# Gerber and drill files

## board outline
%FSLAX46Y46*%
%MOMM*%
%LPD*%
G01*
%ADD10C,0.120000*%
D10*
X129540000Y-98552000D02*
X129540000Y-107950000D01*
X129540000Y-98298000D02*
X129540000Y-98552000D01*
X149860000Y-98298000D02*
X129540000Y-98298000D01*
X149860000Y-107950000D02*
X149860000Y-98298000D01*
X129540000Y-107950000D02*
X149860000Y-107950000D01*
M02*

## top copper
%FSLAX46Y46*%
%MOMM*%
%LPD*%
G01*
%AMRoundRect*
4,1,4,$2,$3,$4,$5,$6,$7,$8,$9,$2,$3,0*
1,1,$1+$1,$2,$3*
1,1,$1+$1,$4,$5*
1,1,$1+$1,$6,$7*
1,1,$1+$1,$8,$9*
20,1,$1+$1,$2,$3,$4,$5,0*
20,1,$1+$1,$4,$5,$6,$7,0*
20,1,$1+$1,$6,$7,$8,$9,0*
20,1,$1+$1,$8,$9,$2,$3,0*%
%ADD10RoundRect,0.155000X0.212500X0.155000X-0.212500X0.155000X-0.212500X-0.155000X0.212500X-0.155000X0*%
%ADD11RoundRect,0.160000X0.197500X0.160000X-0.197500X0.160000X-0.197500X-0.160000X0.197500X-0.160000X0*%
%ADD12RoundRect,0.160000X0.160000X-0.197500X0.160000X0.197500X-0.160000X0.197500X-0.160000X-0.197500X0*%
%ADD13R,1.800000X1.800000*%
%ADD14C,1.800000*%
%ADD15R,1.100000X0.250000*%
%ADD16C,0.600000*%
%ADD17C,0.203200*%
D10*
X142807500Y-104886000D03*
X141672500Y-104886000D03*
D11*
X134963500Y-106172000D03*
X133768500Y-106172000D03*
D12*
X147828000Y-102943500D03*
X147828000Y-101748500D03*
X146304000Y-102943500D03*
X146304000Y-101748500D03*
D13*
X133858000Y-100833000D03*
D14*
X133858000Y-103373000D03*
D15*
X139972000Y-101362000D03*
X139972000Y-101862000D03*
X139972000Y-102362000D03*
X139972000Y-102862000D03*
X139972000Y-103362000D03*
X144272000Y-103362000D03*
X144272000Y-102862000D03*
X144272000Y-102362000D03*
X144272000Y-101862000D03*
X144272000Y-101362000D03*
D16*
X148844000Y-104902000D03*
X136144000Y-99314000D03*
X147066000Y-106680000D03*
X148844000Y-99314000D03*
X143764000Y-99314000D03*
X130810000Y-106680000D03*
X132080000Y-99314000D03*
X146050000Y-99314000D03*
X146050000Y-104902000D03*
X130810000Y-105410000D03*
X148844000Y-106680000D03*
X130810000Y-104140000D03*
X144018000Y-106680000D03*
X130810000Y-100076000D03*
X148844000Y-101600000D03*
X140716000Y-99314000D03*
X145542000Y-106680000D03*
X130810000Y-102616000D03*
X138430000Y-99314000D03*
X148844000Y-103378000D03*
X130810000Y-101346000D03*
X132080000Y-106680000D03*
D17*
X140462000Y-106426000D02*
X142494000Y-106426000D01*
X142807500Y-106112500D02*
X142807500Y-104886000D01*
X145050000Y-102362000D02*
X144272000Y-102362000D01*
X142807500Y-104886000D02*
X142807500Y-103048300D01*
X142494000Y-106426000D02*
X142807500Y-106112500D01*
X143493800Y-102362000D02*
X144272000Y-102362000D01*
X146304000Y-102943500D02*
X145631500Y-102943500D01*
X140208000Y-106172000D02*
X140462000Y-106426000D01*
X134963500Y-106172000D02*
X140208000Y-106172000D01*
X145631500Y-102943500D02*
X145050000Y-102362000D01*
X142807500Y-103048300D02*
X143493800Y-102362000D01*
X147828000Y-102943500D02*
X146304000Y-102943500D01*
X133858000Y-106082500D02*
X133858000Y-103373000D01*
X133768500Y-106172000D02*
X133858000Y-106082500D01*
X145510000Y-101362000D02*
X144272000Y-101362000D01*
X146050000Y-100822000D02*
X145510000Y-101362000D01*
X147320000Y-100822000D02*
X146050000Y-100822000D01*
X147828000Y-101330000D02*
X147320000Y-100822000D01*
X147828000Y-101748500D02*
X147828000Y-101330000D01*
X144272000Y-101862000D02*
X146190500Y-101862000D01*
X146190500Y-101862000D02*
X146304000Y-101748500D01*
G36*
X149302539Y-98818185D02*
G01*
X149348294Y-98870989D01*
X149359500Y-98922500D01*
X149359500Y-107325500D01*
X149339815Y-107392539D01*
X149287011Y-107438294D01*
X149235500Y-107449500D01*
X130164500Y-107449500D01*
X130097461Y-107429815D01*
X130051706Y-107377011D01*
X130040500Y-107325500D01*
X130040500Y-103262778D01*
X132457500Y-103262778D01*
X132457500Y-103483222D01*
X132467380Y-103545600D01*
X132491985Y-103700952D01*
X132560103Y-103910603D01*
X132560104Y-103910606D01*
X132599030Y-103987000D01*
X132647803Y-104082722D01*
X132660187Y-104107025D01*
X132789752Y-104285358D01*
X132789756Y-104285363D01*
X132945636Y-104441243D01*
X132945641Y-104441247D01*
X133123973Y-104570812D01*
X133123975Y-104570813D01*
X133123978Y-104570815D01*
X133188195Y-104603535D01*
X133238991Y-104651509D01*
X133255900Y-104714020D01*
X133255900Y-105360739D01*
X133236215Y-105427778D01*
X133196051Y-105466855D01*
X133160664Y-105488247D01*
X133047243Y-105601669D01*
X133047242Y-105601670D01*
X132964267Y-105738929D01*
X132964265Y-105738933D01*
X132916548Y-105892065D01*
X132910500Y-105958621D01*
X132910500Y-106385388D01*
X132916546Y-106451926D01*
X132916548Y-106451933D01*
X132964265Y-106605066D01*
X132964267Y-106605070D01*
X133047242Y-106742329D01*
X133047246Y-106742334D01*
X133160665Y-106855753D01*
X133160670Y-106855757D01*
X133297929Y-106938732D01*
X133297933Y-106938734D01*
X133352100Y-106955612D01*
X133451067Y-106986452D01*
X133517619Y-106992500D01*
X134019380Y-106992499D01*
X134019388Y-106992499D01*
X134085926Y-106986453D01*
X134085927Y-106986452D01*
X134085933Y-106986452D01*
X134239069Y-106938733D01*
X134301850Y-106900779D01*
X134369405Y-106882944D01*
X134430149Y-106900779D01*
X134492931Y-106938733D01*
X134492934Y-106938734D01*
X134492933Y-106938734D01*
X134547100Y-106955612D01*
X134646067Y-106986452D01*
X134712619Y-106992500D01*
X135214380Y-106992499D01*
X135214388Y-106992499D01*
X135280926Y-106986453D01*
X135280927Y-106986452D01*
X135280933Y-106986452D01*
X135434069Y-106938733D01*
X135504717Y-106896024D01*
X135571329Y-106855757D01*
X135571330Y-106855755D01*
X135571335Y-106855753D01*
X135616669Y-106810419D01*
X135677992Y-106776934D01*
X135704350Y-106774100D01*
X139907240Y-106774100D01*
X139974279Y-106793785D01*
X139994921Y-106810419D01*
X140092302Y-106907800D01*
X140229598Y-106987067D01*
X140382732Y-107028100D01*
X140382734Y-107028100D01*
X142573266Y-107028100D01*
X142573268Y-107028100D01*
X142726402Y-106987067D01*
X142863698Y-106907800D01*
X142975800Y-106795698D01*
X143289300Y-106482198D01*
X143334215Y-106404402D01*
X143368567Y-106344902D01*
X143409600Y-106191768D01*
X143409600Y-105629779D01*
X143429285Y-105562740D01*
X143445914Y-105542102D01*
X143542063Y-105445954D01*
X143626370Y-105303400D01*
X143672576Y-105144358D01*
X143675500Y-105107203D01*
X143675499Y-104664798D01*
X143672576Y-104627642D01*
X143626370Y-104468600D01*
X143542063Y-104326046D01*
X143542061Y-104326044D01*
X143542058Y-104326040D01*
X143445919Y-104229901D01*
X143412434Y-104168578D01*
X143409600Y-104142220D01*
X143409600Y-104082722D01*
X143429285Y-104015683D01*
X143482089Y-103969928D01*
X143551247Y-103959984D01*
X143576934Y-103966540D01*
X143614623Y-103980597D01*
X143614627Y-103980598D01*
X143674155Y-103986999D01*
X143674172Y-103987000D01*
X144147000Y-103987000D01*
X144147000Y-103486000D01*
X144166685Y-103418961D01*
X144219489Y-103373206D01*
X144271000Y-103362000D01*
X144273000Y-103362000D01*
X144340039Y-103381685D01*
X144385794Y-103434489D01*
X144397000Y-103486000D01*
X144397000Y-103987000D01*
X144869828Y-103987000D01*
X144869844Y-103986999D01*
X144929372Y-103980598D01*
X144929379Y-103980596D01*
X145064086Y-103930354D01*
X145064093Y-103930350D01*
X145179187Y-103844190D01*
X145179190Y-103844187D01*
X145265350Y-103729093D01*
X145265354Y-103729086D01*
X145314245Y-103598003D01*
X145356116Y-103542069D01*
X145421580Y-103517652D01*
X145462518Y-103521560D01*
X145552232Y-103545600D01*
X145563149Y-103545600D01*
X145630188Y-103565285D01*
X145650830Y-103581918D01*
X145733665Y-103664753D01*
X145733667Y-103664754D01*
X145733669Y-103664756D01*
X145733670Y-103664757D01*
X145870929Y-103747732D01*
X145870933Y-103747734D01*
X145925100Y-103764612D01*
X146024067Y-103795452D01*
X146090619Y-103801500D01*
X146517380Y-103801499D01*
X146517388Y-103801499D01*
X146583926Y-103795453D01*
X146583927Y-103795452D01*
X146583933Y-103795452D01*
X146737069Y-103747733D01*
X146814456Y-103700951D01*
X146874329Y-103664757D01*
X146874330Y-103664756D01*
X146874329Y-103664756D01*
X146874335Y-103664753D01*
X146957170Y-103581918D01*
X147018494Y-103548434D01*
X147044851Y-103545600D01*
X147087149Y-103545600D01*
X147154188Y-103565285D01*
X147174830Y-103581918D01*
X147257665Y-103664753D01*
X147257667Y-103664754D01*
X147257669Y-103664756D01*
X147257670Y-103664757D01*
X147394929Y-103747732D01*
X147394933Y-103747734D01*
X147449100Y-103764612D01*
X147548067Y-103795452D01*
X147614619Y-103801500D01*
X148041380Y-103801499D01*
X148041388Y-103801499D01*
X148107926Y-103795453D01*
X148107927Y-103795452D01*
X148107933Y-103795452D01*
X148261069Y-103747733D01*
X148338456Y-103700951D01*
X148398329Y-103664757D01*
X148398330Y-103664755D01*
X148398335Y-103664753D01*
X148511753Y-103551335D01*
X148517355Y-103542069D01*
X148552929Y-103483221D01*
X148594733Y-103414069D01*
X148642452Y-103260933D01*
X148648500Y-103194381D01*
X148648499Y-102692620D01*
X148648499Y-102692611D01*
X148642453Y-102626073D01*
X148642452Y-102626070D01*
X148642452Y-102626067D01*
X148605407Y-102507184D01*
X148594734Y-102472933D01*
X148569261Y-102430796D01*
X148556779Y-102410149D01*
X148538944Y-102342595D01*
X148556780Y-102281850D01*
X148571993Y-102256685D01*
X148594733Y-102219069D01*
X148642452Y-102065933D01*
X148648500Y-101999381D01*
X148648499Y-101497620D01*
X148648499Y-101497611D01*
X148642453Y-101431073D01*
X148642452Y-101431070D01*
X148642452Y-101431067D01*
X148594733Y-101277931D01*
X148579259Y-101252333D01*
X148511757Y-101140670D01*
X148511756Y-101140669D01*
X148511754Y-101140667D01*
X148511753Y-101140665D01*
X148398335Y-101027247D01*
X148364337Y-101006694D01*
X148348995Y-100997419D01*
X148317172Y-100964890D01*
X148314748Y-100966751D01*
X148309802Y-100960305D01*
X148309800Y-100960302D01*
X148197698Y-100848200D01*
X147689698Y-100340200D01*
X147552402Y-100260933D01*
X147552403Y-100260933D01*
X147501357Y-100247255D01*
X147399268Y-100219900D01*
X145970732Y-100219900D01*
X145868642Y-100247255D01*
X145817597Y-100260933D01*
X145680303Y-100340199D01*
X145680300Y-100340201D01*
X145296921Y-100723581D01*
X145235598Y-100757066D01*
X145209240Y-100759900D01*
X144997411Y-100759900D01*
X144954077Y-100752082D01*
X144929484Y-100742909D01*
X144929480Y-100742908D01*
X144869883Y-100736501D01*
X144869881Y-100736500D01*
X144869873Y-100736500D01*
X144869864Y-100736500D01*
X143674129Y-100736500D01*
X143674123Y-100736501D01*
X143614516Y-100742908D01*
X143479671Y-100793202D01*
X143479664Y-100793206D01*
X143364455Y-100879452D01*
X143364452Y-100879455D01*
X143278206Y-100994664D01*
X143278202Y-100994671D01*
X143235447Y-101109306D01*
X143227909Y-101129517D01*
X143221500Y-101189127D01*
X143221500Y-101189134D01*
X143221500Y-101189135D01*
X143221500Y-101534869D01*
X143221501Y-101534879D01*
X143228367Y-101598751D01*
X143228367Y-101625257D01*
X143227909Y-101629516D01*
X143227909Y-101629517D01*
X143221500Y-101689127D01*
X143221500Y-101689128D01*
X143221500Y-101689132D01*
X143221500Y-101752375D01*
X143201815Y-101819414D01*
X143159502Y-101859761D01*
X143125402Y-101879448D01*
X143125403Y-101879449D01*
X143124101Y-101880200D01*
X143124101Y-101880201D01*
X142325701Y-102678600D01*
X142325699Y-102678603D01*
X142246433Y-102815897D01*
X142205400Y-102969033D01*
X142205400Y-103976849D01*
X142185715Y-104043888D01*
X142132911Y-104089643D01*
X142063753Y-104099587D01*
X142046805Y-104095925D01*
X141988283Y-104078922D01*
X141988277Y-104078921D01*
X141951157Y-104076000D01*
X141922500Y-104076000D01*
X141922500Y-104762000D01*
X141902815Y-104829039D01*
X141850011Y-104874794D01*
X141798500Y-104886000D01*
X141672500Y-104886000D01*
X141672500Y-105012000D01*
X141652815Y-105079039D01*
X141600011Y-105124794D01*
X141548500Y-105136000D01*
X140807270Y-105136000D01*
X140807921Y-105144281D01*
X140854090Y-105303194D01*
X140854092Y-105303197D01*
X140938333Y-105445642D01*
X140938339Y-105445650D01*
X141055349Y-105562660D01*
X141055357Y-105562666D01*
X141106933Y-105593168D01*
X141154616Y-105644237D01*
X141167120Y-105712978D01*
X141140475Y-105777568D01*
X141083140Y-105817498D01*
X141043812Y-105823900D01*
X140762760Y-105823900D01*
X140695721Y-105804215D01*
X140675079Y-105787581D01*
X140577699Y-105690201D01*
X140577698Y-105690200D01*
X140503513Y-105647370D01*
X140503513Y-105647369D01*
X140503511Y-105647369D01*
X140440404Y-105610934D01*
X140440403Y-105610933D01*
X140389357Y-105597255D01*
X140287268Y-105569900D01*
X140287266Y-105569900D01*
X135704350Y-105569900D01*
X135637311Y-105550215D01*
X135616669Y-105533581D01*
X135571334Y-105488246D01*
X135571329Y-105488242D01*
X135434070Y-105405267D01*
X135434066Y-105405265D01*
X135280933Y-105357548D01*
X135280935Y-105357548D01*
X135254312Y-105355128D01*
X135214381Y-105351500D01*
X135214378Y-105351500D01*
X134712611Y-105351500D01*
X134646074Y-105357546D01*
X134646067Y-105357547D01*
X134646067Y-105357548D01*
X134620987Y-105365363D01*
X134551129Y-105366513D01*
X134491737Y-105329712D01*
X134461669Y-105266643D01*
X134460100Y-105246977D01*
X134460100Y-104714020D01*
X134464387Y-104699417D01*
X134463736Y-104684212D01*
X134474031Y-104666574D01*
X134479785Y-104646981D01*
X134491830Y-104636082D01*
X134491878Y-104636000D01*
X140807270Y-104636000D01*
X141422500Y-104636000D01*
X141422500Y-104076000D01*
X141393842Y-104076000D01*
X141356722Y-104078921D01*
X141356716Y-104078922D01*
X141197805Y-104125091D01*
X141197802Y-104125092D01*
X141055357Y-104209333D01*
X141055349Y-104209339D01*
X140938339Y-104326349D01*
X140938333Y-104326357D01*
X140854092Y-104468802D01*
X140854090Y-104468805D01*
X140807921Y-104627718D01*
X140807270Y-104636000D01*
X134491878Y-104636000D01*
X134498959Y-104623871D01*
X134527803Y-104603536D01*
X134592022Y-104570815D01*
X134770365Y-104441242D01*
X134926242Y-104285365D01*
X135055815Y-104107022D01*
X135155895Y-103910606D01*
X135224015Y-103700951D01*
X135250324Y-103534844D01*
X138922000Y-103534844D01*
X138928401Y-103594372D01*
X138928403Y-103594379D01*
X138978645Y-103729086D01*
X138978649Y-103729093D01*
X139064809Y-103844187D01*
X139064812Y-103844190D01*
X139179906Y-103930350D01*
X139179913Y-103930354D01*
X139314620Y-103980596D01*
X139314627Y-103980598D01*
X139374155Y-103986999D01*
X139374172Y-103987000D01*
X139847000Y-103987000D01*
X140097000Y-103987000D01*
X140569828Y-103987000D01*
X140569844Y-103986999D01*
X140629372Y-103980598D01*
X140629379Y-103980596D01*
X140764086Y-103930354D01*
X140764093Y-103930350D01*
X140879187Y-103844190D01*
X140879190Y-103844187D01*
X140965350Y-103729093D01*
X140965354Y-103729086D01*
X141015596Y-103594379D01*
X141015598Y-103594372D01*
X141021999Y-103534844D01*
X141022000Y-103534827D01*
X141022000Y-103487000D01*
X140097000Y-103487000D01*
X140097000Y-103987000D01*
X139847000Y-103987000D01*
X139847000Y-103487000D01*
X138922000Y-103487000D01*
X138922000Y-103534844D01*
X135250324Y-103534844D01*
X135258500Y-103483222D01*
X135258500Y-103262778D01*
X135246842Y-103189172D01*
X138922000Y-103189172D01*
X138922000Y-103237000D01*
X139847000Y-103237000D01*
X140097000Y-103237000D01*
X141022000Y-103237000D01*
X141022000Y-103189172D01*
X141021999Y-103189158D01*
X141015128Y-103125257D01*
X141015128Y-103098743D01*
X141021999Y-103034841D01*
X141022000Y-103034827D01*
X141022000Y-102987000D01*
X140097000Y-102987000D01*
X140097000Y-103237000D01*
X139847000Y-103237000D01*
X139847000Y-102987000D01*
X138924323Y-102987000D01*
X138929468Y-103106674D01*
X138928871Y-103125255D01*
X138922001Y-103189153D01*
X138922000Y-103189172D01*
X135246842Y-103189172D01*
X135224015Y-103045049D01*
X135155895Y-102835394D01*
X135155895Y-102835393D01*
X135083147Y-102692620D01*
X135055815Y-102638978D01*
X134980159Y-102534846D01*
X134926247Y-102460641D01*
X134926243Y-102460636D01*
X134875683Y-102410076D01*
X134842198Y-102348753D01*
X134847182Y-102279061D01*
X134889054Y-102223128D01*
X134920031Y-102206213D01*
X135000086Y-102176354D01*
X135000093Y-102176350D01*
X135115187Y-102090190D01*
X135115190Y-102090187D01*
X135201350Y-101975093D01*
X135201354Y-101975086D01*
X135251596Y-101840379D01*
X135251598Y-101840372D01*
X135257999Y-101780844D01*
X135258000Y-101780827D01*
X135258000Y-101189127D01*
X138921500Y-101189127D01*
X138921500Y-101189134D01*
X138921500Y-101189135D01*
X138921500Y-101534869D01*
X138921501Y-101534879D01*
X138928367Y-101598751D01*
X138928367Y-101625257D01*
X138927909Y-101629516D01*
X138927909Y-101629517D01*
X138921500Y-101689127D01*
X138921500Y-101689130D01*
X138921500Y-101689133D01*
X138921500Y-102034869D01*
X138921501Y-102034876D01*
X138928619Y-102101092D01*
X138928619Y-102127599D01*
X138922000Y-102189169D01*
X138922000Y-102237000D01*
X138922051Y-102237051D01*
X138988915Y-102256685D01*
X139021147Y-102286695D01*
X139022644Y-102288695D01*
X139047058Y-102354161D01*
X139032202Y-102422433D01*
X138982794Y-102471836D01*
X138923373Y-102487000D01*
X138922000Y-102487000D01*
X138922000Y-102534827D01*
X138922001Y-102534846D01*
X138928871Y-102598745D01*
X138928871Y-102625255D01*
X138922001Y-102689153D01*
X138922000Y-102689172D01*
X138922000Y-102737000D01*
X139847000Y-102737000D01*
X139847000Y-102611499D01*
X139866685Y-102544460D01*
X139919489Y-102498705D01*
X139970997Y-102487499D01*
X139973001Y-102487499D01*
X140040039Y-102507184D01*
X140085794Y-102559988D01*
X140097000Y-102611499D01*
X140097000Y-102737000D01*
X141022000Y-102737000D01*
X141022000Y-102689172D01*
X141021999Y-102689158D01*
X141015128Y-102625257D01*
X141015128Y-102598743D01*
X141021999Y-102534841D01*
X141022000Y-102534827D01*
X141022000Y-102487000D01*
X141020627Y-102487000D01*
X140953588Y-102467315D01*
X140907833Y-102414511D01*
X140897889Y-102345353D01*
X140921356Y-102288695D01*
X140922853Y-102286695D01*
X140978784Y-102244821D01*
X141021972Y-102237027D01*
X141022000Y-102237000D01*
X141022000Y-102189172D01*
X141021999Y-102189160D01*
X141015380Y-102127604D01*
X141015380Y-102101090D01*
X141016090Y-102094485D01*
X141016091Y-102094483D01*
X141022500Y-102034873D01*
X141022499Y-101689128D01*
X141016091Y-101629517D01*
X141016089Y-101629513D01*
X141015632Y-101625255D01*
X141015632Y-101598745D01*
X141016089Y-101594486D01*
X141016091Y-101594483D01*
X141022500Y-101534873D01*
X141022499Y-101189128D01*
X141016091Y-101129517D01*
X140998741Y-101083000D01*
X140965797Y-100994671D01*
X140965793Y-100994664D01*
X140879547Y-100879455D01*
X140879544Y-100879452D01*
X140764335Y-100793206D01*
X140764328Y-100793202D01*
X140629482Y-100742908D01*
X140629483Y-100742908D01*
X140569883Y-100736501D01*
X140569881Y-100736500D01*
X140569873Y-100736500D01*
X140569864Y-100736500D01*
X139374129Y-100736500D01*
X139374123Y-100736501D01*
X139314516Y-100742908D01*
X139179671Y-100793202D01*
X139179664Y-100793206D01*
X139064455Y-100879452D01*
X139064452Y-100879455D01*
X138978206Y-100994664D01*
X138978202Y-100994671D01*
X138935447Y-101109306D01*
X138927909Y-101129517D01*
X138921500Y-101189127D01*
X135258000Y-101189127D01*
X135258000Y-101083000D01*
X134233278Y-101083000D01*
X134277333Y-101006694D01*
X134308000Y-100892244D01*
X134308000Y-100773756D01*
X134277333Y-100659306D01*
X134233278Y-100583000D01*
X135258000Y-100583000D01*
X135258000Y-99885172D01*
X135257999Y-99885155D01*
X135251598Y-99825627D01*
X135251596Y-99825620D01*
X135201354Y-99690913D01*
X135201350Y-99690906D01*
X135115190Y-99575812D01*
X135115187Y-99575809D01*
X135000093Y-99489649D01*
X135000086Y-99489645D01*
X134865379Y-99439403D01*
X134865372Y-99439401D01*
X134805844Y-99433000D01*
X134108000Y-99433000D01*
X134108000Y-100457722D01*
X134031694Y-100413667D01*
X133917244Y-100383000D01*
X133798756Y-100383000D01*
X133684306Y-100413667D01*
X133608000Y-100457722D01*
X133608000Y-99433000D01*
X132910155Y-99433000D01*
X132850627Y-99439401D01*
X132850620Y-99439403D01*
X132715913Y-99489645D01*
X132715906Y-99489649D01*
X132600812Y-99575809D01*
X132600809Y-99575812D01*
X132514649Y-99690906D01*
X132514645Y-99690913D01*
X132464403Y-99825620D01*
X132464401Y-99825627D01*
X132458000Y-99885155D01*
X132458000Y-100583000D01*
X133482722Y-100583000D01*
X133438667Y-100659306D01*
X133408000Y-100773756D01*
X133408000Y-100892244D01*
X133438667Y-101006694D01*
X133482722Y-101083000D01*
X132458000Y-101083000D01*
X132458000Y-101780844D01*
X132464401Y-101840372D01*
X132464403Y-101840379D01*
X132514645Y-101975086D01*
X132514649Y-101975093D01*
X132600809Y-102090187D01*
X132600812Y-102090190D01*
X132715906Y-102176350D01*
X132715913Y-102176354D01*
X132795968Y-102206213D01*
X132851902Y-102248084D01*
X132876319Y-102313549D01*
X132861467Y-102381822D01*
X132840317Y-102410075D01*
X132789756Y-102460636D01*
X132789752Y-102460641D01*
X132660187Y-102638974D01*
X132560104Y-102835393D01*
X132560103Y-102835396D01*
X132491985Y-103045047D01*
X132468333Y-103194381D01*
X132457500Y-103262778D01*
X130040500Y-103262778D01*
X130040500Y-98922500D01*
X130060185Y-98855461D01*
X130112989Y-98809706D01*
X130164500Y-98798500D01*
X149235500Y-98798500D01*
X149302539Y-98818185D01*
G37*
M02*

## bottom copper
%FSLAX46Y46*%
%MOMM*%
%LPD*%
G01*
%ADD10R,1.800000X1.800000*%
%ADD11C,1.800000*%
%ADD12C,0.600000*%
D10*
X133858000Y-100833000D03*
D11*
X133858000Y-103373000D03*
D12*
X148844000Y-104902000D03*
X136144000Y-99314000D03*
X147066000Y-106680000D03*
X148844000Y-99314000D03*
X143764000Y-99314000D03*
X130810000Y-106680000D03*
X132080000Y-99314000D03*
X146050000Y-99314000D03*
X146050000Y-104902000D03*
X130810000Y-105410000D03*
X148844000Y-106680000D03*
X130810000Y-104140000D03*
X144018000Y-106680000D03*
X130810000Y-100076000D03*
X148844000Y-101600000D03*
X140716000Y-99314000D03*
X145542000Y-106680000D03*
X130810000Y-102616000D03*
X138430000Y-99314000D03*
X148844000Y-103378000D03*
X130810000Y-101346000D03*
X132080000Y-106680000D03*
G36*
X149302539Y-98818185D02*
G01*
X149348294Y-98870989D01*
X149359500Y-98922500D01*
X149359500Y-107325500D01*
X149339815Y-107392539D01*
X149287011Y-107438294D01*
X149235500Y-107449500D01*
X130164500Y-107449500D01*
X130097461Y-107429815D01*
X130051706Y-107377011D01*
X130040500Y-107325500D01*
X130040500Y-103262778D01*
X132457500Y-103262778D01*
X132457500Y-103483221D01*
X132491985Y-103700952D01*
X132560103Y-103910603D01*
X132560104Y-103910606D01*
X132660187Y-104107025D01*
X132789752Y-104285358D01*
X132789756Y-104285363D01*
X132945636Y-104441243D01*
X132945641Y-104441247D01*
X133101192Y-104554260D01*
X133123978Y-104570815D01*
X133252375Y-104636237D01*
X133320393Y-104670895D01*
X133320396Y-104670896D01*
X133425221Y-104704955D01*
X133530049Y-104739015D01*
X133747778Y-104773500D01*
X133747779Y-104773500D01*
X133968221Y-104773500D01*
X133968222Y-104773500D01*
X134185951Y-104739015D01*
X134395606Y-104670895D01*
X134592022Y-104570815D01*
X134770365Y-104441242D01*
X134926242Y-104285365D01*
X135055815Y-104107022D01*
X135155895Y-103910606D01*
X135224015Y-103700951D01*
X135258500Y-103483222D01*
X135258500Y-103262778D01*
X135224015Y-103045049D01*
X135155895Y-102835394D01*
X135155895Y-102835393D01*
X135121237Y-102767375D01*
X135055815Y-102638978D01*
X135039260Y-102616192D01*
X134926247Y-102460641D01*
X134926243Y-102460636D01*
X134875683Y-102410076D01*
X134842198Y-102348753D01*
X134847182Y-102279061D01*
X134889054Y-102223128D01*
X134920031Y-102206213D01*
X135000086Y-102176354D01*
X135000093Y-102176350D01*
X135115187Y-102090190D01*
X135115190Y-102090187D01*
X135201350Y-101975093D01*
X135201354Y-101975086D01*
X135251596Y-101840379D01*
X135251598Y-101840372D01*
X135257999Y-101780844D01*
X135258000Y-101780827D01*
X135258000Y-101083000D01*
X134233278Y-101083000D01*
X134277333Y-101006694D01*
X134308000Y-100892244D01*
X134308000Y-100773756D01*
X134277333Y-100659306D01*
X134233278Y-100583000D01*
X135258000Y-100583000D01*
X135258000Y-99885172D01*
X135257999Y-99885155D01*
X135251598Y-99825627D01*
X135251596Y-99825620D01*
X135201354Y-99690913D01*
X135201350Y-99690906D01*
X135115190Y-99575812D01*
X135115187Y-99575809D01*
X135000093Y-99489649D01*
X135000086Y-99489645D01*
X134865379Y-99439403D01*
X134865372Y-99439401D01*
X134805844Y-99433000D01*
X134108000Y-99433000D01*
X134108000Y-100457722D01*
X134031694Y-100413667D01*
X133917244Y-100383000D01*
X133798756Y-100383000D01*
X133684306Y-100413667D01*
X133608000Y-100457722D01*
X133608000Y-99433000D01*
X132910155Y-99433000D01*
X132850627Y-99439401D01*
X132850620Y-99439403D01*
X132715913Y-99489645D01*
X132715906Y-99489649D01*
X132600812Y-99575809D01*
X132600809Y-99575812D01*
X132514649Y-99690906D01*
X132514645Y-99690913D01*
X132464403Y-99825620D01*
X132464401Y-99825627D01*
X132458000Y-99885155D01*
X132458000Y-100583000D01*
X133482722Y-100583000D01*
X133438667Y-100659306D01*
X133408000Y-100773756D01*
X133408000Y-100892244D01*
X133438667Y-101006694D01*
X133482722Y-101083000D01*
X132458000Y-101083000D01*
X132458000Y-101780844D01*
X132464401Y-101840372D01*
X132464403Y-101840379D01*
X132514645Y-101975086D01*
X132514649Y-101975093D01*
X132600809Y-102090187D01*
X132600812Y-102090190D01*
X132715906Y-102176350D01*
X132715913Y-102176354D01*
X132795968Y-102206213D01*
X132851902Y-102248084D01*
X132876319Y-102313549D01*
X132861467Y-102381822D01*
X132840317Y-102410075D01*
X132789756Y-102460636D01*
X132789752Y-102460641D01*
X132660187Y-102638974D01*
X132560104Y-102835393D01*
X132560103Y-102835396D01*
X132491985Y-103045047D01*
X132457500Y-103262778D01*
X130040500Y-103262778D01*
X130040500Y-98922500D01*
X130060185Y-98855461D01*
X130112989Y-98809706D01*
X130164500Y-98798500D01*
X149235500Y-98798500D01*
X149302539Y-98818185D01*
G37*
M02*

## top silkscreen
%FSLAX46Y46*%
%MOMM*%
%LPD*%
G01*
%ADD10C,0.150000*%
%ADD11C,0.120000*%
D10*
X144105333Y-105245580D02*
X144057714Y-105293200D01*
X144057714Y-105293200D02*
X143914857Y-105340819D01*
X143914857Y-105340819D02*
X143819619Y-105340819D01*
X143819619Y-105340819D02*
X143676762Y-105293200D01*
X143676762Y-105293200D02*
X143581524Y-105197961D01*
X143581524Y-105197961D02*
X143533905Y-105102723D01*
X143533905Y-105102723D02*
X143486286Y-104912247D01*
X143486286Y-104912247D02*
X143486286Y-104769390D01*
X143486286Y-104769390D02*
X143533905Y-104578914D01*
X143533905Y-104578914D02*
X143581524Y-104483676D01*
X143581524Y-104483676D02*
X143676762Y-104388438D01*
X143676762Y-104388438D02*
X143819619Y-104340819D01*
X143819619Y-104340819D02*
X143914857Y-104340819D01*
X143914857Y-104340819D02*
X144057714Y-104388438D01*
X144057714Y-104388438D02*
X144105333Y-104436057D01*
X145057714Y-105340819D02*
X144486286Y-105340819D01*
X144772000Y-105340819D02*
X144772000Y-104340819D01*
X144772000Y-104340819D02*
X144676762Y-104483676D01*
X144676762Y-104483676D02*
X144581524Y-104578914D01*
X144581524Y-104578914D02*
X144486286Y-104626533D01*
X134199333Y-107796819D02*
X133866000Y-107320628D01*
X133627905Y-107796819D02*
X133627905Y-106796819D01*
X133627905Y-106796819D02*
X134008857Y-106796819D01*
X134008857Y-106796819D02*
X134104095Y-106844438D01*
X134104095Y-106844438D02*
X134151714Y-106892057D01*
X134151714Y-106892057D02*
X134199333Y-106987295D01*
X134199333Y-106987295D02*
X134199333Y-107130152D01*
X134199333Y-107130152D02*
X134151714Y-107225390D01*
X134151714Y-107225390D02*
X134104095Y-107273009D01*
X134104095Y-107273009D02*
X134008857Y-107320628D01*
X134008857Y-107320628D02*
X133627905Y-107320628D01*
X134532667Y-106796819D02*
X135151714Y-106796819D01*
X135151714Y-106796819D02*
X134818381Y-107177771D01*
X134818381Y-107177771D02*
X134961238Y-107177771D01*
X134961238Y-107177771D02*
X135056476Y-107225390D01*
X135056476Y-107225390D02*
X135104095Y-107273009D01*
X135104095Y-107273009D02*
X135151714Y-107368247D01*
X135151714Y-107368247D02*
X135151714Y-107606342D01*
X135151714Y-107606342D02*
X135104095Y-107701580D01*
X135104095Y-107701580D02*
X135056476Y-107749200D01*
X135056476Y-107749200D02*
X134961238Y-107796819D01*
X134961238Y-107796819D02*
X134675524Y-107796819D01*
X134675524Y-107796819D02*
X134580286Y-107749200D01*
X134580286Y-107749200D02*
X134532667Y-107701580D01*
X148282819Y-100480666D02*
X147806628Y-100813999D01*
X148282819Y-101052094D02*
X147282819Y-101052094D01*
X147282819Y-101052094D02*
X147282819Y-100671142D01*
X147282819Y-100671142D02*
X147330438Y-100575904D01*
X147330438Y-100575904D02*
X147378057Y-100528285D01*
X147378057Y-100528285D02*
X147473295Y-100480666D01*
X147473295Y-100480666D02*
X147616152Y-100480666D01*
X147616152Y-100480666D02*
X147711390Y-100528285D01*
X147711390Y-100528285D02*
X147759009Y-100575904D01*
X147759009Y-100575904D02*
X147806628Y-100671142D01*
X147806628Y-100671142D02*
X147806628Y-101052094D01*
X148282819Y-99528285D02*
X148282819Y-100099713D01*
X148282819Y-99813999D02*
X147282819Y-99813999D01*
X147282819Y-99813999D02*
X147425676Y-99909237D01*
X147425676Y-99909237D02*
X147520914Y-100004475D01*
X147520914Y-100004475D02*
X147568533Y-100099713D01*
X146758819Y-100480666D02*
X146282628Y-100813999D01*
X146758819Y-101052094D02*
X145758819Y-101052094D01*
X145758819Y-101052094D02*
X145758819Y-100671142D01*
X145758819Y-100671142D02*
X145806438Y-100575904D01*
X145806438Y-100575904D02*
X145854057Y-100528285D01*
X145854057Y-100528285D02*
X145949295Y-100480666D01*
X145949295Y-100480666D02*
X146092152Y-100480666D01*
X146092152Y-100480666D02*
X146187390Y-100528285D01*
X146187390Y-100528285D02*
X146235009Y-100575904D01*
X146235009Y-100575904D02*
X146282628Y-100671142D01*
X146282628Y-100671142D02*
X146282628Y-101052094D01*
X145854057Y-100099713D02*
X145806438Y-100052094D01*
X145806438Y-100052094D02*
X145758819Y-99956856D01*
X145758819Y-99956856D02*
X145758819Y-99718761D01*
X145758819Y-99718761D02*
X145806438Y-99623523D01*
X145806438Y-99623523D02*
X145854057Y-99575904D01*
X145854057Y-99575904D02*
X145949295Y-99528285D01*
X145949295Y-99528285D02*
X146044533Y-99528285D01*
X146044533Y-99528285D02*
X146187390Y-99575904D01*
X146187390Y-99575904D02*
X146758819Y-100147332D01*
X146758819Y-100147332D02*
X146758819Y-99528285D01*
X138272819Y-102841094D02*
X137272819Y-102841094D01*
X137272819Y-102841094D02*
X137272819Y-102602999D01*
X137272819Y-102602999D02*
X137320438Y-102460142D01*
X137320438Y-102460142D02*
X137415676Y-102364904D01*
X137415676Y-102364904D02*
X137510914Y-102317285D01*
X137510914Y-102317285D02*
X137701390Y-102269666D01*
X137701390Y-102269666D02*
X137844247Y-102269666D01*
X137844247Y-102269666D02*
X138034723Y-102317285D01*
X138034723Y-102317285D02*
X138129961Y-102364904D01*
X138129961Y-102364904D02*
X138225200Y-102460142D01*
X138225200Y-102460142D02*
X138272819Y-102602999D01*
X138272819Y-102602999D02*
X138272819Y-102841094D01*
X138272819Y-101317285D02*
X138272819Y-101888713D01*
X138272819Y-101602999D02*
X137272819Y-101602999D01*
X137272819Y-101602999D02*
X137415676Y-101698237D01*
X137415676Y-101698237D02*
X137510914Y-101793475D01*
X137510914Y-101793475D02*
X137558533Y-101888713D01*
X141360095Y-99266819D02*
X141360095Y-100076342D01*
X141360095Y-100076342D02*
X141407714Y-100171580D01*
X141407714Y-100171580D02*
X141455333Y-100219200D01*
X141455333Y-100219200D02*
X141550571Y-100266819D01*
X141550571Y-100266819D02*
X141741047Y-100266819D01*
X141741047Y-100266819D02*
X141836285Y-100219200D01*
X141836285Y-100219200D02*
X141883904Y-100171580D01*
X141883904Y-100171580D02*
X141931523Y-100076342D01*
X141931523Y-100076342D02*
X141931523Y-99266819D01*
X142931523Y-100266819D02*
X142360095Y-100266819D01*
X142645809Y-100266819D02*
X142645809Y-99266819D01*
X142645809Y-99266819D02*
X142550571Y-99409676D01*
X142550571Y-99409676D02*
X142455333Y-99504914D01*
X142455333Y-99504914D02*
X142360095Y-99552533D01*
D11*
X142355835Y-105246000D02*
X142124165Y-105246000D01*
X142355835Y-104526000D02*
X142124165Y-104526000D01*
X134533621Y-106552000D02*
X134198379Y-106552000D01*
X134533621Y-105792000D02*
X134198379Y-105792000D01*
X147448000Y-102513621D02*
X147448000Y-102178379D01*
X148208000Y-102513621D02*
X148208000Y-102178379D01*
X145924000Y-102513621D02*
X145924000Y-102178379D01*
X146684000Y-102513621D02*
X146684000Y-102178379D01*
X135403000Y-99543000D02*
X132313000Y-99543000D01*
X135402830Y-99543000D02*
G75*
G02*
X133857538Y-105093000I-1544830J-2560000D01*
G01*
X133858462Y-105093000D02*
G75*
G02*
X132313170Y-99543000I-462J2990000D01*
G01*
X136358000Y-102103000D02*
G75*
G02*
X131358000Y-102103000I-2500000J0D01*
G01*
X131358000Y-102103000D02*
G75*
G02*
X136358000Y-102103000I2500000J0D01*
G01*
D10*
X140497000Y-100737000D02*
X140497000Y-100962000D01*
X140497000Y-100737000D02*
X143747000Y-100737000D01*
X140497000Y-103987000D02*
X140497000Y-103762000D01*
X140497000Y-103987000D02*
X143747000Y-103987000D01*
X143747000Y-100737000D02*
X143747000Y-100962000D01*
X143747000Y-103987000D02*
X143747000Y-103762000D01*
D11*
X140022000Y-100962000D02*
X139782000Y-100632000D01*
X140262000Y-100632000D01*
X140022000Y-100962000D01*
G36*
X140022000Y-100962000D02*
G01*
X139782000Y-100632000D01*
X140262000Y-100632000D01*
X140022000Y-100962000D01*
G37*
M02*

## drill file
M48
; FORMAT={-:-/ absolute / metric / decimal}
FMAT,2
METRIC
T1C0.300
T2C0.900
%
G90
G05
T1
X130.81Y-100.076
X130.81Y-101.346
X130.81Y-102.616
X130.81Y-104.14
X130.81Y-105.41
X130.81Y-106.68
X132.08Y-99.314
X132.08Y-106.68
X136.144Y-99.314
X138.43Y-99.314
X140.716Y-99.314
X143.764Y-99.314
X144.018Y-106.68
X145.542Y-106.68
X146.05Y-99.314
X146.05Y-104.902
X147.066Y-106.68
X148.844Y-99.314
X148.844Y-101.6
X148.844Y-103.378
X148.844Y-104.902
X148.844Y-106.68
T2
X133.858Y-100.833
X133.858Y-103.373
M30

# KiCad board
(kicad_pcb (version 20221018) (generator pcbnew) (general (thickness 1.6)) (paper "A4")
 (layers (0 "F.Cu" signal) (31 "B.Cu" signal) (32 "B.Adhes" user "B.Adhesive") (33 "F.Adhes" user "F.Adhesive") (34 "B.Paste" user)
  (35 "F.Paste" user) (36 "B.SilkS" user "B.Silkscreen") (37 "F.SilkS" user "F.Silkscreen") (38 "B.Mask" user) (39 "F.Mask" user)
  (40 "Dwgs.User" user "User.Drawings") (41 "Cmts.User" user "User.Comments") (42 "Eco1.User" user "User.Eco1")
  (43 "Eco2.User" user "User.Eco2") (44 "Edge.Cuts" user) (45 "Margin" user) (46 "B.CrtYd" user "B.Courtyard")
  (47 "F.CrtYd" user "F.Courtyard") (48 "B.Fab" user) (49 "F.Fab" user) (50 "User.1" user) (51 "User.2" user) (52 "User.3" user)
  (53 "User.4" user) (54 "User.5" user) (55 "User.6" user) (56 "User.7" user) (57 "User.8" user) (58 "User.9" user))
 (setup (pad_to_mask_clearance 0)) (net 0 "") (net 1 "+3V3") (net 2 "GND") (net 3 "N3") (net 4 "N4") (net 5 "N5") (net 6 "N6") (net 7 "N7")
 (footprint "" (layer "F.Cu") (at 142.24 104.886 180)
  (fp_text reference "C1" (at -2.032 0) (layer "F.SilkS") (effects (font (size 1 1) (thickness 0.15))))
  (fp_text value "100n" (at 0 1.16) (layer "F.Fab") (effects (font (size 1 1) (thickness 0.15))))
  (fp_line (start -0.115835 -0.36) (end 0.115835 -0.36) (layer "F.SilkS") (stroke (width 0.12) (type solid)))
  (fp_line (start -0.115835 0.36) (end 0.115835 0.36) (layer "F.SilkS") (stroke (width 0.12) (type solid)))
  (pad "1" smd roundrect (at -0.5675 0 180) (size 0.735 0.62) (layers "F.Cu" "F.Paste" "F.Mask") (roundrect_rratio 0.25) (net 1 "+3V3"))
  (pad "2" smd roundrect (at 0.5675 0 180) (size 0.735 0.62) (layers "F.Cu" "F.Paste" "F.Mask") (roundrect_rratio 0.25) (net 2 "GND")))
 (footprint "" (layer "F.Cu") (at 134.366 106.172 180)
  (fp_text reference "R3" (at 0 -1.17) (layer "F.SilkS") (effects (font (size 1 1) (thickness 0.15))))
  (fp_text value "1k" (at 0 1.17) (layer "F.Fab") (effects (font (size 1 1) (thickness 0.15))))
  (fp_line (start -0.167621 -0.38) (end 0.167621 -0.38) (layer "F.SilkS") (stroke (width 0.12) (type solid)))
  (fp_line (start -0.167621 0.38) (end 0.167621 0.38) (layer "F.SilkS") (stroke (width 0.12) (type solid)))
  (pad "1" smd roundrect (at -0.5975 0 180) (size 0.715 0.64) (layers "F.Cu" "F.Paste" "F.Mask") (roundrect_rratio 0.25) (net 1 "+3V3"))
  (pad "2" smd roundrect (at 0.5975 0 180) (size 0.715 0.64) (layers "F.Cu" "F.Paste" "F.Mask") (roundrect_rratio 0.25) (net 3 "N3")))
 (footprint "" (layer "F.Cu") (at 147.828 102.346 90)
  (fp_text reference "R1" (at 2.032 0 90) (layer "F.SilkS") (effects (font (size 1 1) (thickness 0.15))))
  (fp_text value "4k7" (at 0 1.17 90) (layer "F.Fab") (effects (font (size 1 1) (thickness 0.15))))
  (fp_line (start -0.167621 -0.38) (end 0.167621 -0.38) (layer "F.SilkS") (stroke (width 0.12) (type solid)))
  (fp_line (start -0.167621 0.38) (end 0.167621 0.38) (layer "F.SilkS") (stroke (width 0.12) (type solid)))
  (pad "1" smd roundrect (at -0.5975 0 90) (size 0.715 0.64) (layers "F.Cu" "F.Paste" "F.Mask") (roundrect_rratio 0.25) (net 1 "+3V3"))
  (pad "2" smd roundrect (at 0.5975 0 90) (size 0.715 0.64) (layers "F.Cu" "F.Paste" "F.Mask") (roundrect_rratio 0.25) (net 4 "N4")))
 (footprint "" (layer "F.Cu") (at 146.304 102.346 90)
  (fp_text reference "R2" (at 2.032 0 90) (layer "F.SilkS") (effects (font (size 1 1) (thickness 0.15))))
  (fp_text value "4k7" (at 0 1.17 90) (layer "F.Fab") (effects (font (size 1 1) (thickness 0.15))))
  (fp_line (start -0.167621 -0.38) (end 0.167621 -0.38) (layer "F.SilkS") (stroke (width 0.12) (type solid)))
  (fp_line (start -0.167621 0.38) (end 0.167621 0.38) (layer "F.SilkS") (stroke (width 0.12) (type solid)))
  (pad "1" smd roundrect (at -0.5975 0 90) (size 0.715 0.64) (layers "F.Cu" "F.Paste" "F.Mask") (roundrect_rratio 0.25) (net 1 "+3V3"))
  (pad "2" smd roundrect (at 0.5975 0 90) (size 0.715 0.64) (layers "F.Cu" "F.Paste" "F.Mask") (roundrect_rratio 0.25) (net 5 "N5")))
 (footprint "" (layer "F.Cu") (at 133.858 100.833 -90)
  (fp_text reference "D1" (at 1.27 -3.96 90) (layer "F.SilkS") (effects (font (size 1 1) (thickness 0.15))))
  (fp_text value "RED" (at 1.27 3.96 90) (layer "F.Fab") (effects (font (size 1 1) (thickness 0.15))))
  (fp_line (start -1.29 -1.545) (end -1.29 1.545) (layer "F.SilkS") (stroke (width 0.12) (type solid)))
  (fp_arc (start -1.29 -1.54483) (mid 2.072002 -2.880433) (end 4.26 0.000462) (layer "F.SilkS") (stroke (width 0.12) (type solid)))
  (fp_arc (start 4.26 -0.000462) (mid 2.072002 2.880433) (end -1.29 1.54483) (layer "F.SilkS") (stroke (width 0.12) (type solid)))
  (fp_circle (center 1.27 0) (end 3.77 0) (layer "F.SilkS") (stroke (width 0.12) (type solid)) (fill none))
  (pad "1" thru_hole rect (at 0 0 270) (size 1.8 1.8) (drill 0.9) (layers *.Cu *.Mask) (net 2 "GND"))
  (pad "2" thru_hole circle (at 2.54 0 270) (size 1.8 1.8) (drill 0.9) (layers *.Cu *.Mask) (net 3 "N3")))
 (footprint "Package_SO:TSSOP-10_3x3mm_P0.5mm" (layer "F.Cu") (at 142.122 102.362)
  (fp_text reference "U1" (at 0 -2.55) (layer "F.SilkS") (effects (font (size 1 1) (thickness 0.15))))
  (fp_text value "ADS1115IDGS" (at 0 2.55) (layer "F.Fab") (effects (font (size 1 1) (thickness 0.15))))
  (fp_line (start -1.625 -1.625) (end -1.625 -1.4) (layer "F.SilkS") (stroke (width 0.15) (type solid)))
  (fp_line (start -1.625 -1.625) (end 1.625 -1.625) (layer "F.SilkS") (stroke (width 0.15) (type solid)))
  (fp_line (start -1.625 1.625) (end -1.625 1.4) (layer "F.SilkS") (stroke (width 0.15) (type solid)))
  (fp_line (start -1.625 1.625) (end 1.625 1.625) (layer "F.SilkS") (stroke (width 0.15) (type solid)))
  (fp_line (start 1.625 -1.625) (end 1.625 -1.4) (layer "F.SilkS") (stroke (width 0.15) (type solid)))
  (fp_line (start 1.625 1.625) (end 1.625 1.4) (layer "F.SilkS") (stroke (width 0.15) (type solid)))
  (fp_poly
   (pts (xy -2.1 -1.4) (xy -2.34 -1.73) (xy -1.86 -1.73) (xy -2.1 -1.4)) (layer "F.SilkS") (stroke (width 0.12) (type solid)) (fill solid))
  (pad "1" smd rect (at -2.15 -1) (size 1.1 0.25) (layers "F.Cu" "F.Paste" "F.Mask") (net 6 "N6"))
  (pad "2" smd rect (at -2.15 -0.5) (size 1.1 0.25) (layers "F.Cu" "F.Paste" "F.Mask") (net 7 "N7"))
  (pad "3" smd rect (at -2.15 0) (size 1.1 0.25) (layers "F.Cu" "F.Paste" "F.Mask") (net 2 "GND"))
  (pad "4" smd rect (at -2.15 0.5) (size 1.1 0.25) (layers "F.Cu" "F.Paste" "F.Mask") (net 2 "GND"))
  (pad "5" smd rect (at -2.15 1) (size 1.1 0.25) (layers "F.Cu" "F.Paste" "F.Mask") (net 2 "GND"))
  (pad "6" smd rect (at 2.15 1) (size 1.1 0.25) (layers "F.Cu" "F.Paste" "F.Mask") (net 2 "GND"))
  (pad "7" smd rect (at 2.15 0.5) (size 1.1 0.25) (layers "F.Cu" "F.Paste" "F.Mask") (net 2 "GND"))
  (pad "8" smd rect (at 2.15 0) (size 1.1 0.25) (layers "F.Cu" "F.Paste" "F.Mask") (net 1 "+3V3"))
  (pad "9" smd rect (at 2.15 -0.5) (size 1.1 0.25) (layers "F.Cu" "F.Paste" "F.Mask") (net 5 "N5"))
  (pad "10" smd rect (at 2.15 -1) (size 1.1 0.25) (layers "F.Cu" "F.Paste" "F.Mask") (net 4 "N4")))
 (gr_line (start 129.54 98.552) (end 129.54 107.95) (layer "Edge.Cuts") (width 0.12))
 (gr_line (start 129.54 98.298) (end 129.54 98.552) (layer "Edge.Cuts") (width 0.12))
 (gr_line (start 149.86 98.298) (end 129.54 98.298) (layer "Edge.Cuts") (width 0.12))
 (gr_line (start 149.86 107.95) (end 149.86 98.298) (layer "Edge.Cuts") (width 0.12))
 (gr_line (start 129.54 107.95) (end 149.86 107.95) (layer "Edge.Cuts") (width 0.12))
 (segment (start 140.462 106.426) (end 142.494 106.426) (width 0.2032) (layer "F.Cu") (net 1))
 (segment (start 142.8075 106.1125) (end 142.8075 104.886) (width 0.2032) (layer "F.Cu") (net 1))
 (segment (start 145.05 102.362) (end 144.272 102.362) (width 0.2032) (layer "F.Cu") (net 1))
 (segment (start 142.8075 104.886) (end 142.8075 103.0483) (width 0.2032) (layer "F.Cu") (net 1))
 (segment (start 142.494 106.426) (end 142.8075 106.1125) (width 0.2032) (layer "F.Cu") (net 1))
 (segment (start 143.4938 102.362) (end 144.272 102.362) (width 0.2032) (layer "F.Cu") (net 1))
 (segment (start 146.304 102.9435) (end 145.6315 102.9435) (width 0.2032) (layer "F.Cu") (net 1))
 (segment (start 140.208 106.172) (end 140.462 106.426) (width 0.2032) (layer "F.Cu") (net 1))
 (segment (start 134.9635 106.172) (end 140.208 106.172) (width 0.2032) (layer "F.Cu") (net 1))
 (segment (start 145.6315 102.9435) (end 145.05 102.362) (width 0.2032) (layer "F.Cu") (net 1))
 (segment (start 142.8075 103.0483) (end 143.4938 102.362) (width 0.2032) (layer "F.Cu") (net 1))
 (segment (start 147.828 102.9435) (end 146.304 102.9435) (width 0.2032) (layer "F.Cu") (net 1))
 (via (at 148.844 104.902) (size 0.6) (drill 0.3) (layers "F.Cu" "B.Cu") (free) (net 2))
 (via (at 136.144 99.314) (size 0.6) (drill 0.3) (layers "F.Cu" "B.Cu") (free) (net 2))
 (via (at 147.066 106.68) (size 0.6) (drill 0.3) (layers "F.Cu" "B.Cu") (free) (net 2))
 (via (at 148.844 99.314) (size 0.6) (drill 0.3) (layers "F.Cu" "B.Cu") (free) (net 2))
 (via (at 143.764 99.314) (size 0.6) (drill 0.3) (layers "F.Cu" "B.Cu") (free) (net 2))
 (via (at 130.81 106.68) (size 0.6) (drill 0.3) (layers "F.Cu" "B.Cu") (free) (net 2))
 (via (at 132.08 99.314) (size 0.6) (drill 0.3) (layers "F.Cu" "B.Cu") (free) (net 2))
 (via (at 146.05 99.314) (size 0.6) (drill 0.3) (layers "F.Cu" "B.Cu") (free) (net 2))
 (via (at 146.05 104.902) (size 0.6) (drill 0.3) (layers "F.Cu" "B.Cu") (free) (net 2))
 (via (at 130.81 105.41) (size 0.6) (drill 0.3) (layers "F.Cu" "B.Cu") (free) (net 2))
 (via (at 148.844 106.68) (size 0.6) (drill 0.3) (layers "F.Cu" "B.Cu") (free) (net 2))
 (via (at 130.81 104.14) (size 0.6) (drill 0.3) (layers "F.Cu" "B.Cu") (free) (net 2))
 (via (at 144.018 106.68) (size 0.6) (drill 0.3) (layers "F.Cu" "B.Cu") (free) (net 2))
 (via (at 130.81 100.076) (size 0.6) (drill 0.3) (layers "F.Cu" "B.Cu") (free) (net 2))
 (via (at 148.844 101.6) (size 0.6) (drill 0.3) (layers "F.Cu" "B.Cu") (free) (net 2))
 (via (at 140.716 99.314) (size 0.6) (drill 0.3) (layers "F.Cu" "B.Cu") (free) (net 2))
 (via (at 145.542 106.68) (size 0.6) (drill 0.3) (layers "F.Cu" "B.Cu") (free) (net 2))
 (via (at 130.81 102.616) (size 0.6) (drill 0.3) (layers "F.Cu" "B.Cu") (free) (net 2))
 (via (at 138.43 99.314) (size 0.6) (drill 0.3) (layers "F.Cu" "B.Cu") (free) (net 2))
 (via (at 148.844 103.378) (size 0.6) (drill 0.3) (layers "F.Cu" "B.Cu") (free) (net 2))
 (via (at 130.81 101.346) (size 0.6) (drill 0.3) (layers "F.Cu" "B.Cu") (free) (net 2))
 (via (at 132.08 106.68) (size 0.6) (drill 0.3) (layers "F.Cu" "B.Cu") (free) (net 2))
 (segment (start 133.858 106.0825) (end 133.858 103.373) (width 0.2032) (layer "F.Cu") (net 3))
 (segment (start 133.7685 106.172) (end 133.858 106.0825) (width 0.2032) (layer "F.Cu") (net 3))
 (segment (start 145.51 101.362) (end 144.272 101.362) (width 0.2032) (layer "F.Cu") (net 4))
 (segment (start 146.05 100.822) (end 145.51 101.362) (width 0.2032) (layer "F.Cu") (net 4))
 (segment (start 147.32 100.822) (end 146.05 100.822) (width 0.2032) (layer "F.Cu") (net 4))
 (segment (start 147.828 101.33) (end 147.32 100.822) (width 0.2032) (layer "F.Cu") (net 4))
 (segment (start 147.828 101.7485) (end 147.828 101.33) (width 0.2032) (layer "F.Cu") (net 4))
 (segment (start 144.272 101.862) (end 146.1905 101.862) (width 0.2032) (layer "F.Cu") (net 5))
 (segment (start 146.1905 101.862) (end 146.304 101.7485) (width 0.2032) (layer "F.Cu") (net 5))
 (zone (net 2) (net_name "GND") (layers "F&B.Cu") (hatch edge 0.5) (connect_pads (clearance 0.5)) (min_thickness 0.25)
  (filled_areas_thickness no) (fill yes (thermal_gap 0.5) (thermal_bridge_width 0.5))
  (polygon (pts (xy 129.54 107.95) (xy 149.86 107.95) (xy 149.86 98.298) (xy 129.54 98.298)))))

